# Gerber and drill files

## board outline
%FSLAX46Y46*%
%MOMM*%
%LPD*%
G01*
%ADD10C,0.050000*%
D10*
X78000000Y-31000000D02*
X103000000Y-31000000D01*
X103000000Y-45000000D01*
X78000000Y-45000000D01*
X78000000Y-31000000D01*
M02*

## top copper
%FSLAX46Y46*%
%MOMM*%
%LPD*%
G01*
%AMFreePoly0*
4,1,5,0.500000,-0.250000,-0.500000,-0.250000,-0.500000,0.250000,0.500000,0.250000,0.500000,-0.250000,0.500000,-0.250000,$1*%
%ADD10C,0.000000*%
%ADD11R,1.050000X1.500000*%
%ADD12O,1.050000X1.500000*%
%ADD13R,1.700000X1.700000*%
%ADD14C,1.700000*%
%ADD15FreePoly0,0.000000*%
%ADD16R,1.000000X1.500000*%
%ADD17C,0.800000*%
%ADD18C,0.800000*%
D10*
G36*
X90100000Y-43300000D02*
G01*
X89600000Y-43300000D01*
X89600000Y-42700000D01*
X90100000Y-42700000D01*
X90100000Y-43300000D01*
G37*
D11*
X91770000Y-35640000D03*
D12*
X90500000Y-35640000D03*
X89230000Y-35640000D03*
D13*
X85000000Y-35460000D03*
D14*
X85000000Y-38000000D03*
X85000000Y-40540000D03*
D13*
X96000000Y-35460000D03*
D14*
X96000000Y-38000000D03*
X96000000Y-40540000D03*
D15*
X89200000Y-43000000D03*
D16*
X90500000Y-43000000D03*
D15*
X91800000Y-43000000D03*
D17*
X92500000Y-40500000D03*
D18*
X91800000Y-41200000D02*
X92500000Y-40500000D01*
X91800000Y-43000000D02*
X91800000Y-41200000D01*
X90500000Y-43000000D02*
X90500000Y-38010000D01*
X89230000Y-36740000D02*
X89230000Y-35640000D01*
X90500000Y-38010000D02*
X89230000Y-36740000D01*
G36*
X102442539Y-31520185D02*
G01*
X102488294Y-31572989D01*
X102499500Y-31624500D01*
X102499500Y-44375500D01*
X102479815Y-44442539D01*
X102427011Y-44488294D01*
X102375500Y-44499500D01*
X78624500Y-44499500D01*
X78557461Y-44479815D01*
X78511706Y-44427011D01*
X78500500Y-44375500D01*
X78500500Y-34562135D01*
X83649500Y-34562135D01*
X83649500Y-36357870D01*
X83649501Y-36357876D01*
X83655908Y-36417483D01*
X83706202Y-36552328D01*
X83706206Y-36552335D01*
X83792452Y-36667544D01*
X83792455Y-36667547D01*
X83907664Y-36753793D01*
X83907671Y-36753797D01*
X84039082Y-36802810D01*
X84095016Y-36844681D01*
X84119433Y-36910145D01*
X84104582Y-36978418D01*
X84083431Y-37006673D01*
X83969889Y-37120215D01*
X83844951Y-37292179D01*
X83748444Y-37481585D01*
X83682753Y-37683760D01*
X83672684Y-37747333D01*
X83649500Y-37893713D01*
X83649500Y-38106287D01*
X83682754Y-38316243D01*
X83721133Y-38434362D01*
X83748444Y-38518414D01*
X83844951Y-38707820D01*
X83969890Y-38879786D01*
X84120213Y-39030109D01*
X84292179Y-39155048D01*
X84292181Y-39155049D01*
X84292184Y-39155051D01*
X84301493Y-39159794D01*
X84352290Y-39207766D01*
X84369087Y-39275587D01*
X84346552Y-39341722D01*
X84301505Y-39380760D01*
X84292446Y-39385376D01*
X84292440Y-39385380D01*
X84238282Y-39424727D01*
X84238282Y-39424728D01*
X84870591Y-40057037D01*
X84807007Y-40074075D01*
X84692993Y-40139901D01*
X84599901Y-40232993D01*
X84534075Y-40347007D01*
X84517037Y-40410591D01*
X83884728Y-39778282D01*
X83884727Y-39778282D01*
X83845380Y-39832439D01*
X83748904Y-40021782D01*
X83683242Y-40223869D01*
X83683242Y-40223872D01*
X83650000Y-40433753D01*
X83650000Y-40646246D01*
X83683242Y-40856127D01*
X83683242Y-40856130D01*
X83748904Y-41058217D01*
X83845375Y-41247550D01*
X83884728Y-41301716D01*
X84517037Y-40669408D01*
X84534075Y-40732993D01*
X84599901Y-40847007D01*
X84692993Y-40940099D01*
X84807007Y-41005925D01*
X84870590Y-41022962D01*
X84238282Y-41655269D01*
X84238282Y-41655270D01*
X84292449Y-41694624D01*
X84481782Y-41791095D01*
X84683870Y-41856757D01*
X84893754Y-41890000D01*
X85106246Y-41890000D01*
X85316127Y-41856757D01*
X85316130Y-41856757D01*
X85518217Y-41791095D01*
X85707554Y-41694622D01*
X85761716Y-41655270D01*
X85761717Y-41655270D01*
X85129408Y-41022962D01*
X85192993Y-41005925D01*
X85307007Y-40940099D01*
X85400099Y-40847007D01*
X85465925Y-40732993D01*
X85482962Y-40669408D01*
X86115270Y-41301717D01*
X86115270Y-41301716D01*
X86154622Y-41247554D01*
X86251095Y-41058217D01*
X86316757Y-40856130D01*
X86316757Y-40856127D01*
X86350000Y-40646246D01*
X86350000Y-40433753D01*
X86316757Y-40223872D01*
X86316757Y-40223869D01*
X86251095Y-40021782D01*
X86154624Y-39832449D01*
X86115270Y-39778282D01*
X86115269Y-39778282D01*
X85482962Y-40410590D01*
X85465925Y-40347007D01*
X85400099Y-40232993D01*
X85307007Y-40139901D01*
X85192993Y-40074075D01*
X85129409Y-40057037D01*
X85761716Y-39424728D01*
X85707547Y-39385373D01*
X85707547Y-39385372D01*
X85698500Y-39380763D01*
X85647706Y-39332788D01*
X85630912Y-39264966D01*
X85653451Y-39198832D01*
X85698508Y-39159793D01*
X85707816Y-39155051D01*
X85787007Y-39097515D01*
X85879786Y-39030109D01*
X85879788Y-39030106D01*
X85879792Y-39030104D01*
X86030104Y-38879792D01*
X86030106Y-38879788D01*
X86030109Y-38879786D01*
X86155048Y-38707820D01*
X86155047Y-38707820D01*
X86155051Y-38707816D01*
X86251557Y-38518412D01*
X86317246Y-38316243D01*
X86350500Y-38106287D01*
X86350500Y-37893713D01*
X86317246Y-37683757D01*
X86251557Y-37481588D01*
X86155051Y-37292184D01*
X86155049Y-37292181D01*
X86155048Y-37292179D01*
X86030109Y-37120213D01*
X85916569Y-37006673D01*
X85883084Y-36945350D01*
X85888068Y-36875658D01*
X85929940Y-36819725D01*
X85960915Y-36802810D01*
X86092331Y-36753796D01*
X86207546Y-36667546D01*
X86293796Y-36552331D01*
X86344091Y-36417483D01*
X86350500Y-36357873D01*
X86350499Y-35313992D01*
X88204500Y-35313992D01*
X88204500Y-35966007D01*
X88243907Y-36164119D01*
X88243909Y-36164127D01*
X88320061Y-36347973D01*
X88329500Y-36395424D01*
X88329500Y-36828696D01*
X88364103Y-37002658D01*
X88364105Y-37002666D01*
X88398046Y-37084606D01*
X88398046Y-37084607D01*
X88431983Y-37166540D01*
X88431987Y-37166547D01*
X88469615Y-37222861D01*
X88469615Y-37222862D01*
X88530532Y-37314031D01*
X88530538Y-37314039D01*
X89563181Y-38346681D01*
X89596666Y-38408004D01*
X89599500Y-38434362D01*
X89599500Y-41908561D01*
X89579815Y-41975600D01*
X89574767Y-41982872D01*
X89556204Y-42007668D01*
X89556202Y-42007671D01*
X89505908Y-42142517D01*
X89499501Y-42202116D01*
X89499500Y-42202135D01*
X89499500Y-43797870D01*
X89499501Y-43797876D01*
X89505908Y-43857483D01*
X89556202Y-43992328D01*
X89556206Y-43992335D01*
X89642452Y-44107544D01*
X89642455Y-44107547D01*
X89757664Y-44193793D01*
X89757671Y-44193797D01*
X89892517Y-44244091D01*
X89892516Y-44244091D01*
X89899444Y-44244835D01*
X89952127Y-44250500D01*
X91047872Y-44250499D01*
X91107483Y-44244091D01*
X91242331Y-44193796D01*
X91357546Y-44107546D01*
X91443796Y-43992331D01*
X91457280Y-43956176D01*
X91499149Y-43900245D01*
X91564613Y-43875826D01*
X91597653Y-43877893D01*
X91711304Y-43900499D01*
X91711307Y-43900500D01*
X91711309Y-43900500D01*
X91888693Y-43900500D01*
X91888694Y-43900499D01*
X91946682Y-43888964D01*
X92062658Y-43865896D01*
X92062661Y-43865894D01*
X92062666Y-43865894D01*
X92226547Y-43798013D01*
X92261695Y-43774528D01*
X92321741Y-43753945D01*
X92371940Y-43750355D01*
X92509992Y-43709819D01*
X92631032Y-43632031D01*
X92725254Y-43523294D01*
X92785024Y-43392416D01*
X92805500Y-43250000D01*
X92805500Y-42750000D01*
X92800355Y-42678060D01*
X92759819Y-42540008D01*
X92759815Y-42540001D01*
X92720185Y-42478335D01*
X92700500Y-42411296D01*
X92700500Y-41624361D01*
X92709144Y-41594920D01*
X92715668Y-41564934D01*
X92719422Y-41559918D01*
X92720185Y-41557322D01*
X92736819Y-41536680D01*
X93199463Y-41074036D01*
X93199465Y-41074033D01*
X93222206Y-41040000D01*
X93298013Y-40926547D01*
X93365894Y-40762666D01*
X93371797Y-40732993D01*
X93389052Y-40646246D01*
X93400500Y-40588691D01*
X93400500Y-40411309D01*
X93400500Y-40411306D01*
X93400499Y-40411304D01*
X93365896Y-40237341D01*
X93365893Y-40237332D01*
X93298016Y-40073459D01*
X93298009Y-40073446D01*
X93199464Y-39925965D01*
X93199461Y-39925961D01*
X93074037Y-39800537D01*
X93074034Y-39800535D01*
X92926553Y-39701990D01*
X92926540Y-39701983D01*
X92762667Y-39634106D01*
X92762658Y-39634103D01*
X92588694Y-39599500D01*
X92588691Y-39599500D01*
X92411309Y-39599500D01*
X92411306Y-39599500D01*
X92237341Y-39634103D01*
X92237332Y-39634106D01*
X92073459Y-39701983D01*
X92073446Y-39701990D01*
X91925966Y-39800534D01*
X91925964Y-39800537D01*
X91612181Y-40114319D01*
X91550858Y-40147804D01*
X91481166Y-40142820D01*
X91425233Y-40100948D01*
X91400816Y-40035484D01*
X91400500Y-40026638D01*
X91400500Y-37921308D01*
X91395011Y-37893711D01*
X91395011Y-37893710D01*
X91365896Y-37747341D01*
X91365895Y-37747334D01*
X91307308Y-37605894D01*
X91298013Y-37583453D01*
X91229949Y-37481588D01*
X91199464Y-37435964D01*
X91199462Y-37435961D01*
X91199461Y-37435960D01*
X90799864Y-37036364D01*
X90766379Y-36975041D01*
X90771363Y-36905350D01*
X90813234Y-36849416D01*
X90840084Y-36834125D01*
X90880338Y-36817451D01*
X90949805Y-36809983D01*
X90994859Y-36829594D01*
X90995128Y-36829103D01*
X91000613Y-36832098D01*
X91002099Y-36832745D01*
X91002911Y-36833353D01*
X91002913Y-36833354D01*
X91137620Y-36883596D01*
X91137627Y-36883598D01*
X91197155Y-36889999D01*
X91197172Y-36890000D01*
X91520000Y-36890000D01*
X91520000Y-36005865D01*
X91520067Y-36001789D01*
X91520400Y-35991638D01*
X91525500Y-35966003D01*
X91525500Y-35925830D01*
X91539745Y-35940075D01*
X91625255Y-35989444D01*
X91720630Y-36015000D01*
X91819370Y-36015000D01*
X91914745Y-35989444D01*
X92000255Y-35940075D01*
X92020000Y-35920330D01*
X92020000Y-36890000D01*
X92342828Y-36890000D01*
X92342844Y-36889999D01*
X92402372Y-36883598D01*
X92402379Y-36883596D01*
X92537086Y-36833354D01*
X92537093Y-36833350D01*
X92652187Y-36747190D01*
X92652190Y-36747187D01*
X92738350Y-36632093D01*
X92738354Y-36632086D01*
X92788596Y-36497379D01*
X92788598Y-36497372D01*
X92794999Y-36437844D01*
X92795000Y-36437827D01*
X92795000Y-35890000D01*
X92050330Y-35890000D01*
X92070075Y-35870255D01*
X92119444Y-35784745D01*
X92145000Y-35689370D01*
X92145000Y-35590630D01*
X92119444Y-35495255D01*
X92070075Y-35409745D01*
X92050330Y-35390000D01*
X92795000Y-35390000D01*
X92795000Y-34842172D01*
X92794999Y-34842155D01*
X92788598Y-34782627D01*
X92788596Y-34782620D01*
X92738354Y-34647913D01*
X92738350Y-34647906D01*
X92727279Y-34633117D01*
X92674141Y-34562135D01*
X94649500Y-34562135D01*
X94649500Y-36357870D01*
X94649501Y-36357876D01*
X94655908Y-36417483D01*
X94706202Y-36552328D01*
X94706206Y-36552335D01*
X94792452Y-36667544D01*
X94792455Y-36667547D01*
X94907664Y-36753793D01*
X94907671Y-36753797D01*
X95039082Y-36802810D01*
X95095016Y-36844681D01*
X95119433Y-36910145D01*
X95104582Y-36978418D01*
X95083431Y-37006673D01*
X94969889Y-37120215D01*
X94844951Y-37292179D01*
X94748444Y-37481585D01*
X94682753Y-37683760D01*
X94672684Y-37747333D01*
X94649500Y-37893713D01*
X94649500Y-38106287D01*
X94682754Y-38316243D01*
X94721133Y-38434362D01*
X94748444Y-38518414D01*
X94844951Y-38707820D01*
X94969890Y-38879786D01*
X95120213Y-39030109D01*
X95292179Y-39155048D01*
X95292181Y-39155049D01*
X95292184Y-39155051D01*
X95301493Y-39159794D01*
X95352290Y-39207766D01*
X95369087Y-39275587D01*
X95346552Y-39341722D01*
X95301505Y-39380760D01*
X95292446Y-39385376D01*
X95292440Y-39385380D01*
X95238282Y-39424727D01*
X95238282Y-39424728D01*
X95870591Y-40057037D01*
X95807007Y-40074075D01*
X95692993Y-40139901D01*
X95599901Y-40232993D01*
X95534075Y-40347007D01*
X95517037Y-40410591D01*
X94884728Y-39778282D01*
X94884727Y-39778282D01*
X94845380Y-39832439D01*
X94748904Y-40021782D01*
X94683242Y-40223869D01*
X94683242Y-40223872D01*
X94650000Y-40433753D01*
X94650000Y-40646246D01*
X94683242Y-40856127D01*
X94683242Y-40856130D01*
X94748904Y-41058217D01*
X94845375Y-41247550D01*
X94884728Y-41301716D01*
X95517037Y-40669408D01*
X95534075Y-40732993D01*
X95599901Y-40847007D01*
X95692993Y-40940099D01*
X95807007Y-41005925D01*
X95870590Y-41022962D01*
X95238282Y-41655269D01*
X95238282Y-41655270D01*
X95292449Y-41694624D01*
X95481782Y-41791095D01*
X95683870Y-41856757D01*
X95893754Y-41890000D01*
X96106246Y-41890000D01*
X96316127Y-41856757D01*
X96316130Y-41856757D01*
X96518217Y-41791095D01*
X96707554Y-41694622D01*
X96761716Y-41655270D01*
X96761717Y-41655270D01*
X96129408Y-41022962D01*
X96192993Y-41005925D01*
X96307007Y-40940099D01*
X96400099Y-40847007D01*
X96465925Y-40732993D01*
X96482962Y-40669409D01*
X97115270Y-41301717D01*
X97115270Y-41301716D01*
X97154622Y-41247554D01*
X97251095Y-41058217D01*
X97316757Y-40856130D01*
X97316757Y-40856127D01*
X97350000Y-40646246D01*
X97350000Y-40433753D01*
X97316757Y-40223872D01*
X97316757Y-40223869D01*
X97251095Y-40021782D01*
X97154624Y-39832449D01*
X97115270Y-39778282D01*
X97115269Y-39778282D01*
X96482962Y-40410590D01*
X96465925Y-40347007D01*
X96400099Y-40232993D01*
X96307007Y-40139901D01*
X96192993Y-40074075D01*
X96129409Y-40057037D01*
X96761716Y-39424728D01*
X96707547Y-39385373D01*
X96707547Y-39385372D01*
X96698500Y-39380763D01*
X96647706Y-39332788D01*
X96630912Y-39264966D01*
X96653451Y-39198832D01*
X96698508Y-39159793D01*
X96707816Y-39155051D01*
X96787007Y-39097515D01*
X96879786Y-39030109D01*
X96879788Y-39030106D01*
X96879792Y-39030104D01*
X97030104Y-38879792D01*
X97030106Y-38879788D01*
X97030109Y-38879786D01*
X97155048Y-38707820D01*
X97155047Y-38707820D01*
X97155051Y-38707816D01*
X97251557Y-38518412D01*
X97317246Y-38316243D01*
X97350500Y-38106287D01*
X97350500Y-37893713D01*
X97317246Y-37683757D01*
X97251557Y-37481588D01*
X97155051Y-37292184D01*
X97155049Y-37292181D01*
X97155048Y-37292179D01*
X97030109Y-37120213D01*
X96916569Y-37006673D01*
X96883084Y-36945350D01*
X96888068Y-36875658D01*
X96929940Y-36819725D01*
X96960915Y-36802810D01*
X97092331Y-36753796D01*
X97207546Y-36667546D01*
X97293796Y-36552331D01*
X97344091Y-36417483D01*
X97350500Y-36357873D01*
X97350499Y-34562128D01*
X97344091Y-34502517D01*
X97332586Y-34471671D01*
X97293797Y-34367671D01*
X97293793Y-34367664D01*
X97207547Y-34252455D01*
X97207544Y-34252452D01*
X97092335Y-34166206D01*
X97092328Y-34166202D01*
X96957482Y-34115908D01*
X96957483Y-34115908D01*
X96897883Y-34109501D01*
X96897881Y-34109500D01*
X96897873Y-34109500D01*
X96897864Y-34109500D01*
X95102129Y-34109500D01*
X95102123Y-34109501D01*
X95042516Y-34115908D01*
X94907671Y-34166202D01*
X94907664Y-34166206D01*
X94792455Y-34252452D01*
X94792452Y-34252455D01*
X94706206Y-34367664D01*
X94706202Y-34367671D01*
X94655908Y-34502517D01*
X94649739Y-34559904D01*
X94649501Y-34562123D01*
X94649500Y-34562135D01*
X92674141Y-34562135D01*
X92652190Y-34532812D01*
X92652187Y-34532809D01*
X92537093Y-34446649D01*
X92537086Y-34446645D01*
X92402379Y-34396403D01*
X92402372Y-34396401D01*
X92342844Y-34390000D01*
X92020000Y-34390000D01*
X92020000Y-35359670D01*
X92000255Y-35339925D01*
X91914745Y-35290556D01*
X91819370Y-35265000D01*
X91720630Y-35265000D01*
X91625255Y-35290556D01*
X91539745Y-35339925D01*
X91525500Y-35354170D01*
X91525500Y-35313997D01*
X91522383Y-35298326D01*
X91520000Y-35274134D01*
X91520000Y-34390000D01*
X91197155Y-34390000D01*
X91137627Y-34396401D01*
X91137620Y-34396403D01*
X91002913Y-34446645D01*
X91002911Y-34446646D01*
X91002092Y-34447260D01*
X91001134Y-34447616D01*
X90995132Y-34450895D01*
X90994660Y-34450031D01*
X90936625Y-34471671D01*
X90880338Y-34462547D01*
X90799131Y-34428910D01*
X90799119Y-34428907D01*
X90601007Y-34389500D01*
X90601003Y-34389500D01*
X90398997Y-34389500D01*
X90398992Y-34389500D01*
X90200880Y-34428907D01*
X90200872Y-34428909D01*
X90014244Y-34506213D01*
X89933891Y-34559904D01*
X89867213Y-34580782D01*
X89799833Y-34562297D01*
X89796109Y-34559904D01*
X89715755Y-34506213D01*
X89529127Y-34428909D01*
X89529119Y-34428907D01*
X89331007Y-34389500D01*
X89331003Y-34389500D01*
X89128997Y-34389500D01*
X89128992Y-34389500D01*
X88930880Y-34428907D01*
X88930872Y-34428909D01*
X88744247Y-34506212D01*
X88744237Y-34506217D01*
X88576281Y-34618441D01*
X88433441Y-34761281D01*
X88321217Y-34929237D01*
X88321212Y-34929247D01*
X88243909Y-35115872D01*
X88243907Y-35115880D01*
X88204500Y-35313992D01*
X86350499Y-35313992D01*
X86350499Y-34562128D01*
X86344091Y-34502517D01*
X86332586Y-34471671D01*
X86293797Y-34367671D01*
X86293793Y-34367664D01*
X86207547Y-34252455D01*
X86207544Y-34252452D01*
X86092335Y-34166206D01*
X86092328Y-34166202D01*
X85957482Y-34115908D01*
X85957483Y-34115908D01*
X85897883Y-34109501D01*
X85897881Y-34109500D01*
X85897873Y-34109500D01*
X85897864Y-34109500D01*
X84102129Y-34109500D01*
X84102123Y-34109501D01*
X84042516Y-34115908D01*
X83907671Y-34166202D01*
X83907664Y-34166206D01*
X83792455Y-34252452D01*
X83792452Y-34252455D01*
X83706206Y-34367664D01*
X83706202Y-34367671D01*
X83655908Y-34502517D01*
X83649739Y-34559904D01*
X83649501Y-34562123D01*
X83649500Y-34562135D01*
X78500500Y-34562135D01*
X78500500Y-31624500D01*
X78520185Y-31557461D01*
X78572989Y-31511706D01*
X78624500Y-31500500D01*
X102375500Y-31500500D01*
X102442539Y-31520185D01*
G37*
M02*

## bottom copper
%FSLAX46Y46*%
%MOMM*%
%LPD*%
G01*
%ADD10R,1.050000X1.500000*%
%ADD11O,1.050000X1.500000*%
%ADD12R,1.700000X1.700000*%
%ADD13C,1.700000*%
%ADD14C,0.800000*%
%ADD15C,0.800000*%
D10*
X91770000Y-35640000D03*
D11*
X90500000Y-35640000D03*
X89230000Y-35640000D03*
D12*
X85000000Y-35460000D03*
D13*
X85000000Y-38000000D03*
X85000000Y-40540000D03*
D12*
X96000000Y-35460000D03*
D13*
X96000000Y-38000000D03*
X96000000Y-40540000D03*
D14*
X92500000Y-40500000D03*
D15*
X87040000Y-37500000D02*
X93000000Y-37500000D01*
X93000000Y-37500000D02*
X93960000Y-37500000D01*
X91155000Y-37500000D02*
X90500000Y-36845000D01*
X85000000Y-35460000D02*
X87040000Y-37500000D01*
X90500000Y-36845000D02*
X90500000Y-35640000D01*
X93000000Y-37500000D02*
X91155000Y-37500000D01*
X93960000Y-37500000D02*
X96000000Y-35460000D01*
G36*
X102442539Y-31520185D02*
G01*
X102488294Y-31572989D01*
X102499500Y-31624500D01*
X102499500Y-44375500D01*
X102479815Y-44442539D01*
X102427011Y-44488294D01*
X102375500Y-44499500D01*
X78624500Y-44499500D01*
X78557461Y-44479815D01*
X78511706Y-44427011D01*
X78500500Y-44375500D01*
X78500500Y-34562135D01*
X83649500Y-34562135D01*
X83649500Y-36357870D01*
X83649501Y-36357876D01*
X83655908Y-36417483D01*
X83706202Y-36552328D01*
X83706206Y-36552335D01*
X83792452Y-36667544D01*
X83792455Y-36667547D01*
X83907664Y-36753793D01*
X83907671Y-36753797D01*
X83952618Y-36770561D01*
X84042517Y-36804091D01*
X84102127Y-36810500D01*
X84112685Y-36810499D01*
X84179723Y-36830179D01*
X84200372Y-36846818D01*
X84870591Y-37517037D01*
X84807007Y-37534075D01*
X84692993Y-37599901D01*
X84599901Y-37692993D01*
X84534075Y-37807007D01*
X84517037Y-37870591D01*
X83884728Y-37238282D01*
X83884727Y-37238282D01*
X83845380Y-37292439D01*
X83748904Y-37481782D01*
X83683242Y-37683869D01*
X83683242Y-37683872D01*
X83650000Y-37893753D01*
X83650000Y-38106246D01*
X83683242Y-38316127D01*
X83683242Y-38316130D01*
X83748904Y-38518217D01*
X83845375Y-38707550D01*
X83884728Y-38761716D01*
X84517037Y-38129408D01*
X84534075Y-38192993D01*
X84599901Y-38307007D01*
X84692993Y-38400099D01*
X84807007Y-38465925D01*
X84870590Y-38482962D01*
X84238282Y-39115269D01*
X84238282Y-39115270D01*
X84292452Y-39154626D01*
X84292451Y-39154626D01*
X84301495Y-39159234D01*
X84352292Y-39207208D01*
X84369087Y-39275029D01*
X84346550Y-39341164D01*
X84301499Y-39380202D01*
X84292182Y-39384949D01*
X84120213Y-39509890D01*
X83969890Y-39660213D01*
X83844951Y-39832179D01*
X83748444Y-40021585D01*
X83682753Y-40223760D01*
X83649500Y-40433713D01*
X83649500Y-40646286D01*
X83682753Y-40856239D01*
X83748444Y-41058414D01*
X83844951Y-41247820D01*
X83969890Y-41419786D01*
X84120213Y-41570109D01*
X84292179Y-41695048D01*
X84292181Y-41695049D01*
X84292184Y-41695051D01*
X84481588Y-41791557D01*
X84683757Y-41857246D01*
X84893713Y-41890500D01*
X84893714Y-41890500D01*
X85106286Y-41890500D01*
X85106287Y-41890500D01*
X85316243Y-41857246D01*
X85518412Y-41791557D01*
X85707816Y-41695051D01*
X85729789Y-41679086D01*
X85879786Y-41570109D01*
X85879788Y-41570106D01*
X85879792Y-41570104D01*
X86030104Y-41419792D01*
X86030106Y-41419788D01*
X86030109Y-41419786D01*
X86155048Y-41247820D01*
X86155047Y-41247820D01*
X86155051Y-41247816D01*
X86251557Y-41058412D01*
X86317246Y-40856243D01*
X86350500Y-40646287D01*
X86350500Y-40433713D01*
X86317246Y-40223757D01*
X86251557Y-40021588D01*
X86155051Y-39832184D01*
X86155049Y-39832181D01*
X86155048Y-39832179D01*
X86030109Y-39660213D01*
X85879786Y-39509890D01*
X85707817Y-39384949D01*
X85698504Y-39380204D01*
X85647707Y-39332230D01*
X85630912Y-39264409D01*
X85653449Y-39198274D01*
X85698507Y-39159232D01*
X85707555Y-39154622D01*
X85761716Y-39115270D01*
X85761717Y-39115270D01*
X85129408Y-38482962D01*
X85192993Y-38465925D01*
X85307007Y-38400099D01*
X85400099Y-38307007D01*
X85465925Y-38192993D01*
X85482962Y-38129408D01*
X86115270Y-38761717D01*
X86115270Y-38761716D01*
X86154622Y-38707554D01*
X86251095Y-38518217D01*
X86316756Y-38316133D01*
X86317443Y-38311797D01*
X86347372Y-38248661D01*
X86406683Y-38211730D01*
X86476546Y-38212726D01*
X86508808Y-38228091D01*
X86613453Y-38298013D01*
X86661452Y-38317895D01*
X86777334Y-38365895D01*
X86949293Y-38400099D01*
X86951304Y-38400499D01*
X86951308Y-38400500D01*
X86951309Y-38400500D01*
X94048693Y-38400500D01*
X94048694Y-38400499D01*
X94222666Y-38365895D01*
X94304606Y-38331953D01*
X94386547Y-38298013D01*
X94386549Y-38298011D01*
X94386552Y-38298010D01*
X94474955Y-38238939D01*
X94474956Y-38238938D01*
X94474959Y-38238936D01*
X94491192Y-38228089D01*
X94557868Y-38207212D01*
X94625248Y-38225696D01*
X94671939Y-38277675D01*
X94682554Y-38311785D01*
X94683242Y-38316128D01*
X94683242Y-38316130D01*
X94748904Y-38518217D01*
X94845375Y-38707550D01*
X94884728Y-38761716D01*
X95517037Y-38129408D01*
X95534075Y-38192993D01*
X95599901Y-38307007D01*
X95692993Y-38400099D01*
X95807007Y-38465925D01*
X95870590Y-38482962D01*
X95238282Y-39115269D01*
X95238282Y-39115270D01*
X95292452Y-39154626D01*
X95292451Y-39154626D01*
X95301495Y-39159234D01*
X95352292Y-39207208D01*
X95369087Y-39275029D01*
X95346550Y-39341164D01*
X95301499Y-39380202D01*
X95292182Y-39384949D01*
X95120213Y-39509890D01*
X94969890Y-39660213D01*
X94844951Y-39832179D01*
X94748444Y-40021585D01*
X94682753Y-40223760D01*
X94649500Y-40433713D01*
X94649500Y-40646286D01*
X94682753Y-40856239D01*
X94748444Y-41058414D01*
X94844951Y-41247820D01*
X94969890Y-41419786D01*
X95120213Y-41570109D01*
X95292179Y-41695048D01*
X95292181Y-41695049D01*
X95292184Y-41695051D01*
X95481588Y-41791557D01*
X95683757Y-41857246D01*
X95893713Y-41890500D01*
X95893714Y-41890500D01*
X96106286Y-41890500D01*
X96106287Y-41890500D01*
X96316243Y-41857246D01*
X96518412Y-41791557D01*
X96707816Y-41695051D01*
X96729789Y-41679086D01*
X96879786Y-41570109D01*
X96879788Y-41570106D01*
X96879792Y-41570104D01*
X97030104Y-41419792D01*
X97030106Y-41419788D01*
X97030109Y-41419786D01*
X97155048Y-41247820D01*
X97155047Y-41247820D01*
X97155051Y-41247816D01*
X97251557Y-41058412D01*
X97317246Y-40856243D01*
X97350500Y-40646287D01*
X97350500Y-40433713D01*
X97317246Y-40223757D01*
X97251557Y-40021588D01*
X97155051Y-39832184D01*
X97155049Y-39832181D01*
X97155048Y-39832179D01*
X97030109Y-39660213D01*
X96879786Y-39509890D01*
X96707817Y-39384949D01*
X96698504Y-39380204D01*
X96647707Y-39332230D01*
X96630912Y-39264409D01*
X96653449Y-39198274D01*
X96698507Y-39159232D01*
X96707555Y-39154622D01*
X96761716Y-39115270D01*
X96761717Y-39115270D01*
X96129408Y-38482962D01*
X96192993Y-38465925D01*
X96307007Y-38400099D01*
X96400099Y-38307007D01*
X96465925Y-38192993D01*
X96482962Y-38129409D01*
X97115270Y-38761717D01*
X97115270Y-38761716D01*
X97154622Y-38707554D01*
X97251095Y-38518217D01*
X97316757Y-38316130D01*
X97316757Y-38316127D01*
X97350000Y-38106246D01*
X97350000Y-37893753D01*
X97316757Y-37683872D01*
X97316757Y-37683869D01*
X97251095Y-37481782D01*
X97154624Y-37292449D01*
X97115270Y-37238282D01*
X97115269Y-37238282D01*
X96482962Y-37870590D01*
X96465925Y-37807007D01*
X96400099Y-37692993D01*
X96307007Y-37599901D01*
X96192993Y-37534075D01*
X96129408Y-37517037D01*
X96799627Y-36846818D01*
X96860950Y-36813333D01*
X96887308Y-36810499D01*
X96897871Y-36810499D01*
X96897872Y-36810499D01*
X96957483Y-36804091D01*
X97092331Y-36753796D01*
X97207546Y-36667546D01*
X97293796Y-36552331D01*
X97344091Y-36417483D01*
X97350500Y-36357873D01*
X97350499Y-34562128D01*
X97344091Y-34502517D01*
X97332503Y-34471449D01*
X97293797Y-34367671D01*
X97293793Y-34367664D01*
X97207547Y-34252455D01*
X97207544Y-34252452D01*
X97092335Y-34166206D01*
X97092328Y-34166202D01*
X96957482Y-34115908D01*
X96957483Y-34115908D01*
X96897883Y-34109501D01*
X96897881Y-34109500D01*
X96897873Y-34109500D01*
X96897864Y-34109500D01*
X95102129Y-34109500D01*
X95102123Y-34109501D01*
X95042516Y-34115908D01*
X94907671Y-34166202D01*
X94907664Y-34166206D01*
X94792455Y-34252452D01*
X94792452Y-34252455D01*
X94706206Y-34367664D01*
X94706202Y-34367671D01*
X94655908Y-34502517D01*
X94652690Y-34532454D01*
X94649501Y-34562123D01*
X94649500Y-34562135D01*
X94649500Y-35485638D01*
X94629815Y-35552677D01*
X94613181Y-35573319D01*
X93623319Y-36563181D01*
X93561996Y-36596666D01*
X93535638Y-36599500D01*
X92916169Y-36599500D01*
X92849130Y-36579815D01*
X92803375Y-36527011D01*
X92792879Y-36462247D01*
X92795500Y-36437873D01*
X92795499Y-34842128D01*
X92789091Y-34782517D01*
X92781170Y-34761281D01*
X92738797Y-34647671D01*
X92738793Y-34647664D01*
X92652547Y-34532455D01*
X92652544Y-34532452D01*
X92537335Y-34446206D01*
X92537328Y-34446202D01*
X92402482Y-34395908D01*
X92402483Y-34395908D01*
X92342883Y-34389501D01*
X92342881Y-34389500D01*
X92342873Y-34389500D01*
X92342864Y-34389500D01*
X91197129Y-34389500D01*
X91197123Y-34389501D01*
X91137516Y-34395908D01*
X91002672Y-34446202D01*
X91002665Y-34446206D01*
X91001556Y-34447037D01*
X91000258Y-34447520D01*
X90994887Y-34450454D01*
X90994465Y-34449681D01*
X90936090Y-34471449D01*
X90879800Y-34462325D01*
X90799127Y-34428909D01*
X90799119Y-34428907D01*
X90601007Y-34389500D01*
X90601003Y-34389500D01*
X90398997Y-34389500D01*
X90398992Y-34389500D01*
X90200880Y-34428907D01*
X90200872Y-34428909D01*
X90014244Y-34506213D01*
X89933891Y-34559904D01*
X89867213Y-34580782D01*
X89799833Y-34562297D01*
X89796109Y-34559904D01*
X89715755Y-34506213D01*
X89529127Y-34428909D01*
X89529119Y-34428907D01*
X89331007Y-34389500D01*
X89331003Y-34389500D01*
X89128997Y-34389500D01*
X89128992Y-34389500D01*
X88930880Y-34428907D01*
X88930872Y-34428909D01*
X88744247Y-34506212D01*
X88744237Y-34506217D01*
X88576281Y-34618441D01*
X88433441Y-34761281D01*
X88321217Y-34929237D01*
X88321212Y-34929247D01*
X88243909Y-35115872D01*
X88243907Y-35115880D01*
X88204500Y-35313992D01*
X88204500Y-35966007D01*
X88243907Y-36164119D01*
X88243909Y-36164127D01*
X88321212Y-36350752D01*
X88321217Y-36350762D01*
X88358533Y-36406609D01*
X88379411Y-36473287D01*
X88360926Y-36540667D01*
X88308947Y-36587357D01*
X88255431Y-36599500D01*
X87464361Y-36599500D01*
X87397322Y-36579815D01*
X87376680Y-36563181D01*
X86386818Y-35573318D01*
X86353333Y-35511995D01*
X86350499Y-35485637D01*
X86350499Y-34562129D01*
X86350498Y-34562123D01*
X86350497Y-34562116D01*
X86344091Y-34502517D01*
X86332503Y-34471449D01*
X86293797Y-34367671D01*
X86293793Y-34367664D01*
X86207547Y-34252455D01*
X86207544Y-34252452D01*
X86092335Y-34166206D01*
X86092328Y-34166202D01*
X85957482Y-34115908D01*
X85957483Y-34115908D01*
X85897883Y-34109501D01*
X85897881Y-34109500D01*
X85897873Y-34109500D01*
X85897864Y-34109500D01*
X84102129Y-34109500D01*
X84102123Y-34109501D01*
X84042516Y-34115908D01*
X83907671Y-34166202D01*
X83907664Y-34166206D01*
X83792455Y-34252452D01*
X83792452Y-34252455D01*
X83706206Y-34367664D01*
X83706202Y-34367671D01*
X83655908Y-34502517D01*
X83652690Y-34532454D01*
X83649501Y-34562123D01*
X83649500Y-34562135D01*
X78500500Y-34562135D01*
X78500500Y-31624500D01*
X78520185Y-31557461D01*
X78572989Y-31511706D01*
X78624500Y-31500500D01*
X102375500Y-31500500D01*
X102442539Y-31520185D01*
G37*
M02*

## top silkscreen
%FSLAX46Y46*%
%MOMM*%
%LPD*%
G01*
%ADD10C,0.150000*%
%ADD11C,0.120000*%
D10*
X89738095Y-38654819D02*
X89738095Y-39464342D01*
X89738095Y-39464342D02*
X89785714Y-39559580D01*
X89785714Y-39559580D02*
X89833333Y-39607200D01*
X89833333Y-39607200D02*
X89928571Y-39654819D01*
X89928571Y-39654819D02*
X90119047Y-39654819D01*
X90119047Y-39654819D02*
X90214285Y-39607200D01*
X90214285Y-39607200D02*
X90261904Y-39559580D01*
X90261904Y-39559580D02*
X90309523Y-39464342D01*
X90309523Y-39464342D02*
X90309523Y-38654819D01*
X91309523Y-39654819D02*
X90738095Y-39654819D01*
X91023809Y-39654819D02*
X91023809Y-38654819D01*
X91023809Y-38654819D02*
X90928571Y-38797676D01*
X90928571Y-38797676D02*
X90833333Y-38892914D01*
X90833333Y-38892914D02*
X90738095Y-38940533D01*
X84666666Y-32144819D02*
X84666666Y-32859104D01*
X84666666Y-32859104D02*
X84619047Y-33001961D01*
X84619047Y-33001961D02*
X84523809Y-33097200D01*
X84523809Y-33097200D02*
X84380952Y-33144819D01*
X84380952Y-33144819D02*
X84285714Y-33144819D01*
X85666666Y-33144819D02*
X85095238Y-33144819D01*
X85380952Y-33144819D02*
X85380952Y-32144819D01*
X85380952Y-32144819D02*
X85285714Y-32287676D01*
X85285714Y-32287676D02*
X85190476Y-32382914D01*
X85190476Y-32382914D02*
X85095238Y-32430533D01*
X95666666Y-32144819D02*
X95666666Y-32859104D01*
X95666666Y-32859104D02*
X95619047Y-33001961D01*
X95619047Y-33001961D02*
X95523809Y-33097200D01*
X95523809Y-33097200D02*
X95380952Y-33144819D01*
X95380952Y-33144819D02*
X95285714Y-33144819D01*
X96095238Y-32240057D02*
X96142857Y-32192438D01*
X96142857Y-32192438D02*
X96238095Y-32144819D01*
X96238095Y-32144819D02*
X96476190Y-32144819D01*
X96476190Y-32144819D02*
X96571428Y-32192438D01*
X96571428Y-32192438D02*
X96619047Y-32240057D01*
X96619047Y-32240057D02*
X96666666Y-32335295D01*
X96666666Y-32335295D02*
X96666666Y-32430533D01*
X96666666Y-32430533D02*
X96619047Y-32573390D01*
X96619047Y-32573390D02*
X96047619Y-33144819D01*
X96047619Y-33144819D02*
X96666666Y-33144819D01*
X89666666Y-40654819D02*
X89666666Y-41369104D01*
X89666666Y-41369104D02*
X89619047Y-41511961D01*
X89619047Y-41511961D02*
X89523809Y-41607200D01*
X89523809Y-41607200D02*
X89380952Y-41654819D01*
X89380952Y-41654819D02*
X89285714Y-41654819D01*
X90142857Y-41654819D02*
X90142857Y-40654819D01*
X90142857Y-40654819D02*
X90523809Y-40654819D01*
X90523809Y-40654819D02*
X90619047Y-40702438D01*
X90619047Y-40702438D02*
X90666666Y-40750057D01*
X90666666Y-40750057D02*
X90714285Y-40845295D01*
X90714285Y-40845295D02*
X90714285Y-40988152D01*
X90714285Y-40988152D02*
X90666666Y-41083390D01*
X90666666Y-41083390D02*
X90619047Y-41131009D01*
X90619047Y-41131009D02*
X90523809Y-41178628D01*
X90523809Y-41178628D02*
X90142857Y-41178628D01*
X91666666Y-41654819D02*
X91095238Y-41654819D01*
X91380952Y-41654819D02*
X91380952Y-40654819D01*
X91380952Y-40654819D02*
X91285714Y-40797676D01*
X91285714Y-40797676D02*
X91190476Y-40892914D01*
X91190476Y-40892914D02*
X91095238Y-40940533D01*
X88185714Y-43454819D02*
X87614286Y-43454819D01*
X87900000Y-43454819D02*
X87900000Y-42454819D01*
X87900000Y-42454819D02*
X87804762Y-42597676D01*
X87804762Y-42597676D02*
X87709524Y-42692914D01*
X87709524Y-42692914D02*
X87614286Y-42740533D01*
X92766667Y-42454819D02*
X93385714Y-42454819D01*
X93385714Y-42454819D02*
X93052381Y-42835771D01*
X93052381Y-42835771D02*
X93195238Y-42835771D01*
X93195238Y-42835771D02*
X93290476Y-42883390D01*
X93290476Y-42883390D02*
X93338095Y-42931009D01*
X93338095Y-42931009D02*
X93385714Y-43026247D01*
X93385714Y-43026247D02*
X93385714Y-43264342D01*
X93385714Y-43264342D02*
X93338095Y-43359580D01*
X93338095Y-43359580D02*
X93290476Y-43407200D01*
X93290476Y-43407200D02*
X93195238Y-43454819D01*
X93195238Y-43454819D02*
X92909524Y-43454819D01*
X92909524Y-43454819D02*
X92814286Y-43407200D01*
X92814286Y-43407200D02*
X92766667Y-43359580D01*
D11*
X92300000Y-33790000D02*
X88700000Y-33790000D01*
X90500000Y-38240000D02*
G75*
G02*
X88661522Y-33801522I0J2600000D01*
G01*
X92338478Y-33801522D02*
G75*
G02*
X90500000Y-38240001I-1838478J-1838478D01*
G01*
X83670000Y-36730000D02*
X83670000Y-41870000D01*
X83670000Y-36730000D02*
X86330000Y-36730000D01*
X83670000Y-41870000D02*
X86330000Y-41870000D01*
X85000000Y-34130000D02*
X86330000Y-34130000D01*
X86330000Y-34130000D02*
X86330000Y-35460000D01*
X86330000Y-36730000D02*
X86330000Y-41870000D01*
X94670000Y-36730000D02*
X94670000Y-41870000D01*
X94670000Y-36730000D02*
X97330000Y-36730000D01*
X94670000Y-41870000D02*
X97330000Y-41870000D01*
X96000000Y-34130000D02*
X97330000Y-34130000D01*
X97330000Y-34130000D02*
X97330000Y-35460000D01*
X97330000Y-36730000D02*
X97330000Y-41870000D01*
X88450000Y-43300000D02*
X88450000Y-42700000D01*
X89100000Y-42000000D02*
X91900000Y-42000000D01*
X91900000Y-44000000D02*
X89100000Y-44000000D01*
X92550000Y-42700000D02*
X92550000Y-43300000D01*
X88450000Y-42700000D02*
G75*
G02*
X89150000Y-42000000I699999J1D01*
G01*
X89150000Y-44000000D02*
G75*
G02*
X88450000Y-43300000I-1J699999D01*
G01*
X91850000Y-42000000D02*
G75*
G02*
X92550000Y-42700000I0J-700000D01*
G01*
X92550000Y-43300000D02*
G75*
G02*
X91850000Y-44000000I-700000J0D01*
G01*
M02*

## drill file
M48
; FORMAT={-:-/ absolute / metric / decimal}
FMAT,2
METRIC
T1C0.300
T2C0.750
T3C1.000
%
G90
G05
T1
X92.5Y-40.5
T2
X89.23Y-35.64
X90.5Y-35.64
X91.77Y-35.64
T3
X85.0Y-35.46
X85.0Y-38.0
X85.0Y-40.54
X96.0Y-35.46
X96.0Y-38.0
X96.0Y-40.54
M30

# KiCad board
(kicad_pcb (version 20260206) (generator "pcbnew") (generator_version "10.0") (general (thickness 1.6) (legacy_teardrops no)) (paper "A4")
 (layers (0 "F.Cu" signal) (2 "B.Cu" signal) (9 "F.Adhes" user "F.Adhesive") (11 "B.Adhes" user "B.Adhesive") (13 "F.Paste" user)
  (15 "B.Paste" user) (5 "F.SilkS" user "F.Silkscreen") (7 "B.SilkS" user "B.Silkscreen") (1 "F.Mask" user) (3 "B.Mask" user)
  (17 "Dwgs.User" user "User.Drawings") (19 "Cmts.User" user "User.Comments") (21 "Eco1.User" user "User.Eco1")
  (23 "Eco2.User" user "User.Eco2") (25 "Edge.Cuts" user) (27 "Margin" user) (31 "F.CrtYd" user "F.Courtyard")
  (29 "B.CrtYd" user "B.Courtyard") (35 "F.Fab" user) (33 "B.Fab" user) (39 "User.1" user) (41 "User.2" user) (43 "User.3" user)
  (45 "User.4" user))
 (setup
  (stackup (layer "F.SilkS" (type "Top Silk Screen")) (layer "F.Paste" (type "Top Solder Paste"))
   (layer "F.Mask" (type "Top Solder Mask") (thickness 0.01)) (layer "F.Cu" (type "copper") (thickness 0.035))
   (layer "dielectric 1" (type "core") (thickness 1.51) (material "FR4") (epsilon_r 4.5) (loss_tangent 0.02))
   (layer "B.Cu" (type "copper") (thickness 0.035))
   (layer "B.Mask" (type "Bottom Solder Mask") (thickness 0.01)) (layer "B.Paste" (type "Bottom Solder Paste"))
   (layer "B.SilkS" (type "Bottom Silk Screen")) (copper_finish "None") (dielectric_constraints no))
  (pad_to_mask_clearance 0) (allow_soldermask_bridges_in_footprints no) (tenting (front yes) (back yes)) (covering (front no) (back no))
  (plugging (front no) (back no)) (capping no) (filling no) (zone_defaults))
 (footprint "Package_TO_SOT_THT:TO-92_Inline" (layer "F.Cu") (at 91.77 35.64 180)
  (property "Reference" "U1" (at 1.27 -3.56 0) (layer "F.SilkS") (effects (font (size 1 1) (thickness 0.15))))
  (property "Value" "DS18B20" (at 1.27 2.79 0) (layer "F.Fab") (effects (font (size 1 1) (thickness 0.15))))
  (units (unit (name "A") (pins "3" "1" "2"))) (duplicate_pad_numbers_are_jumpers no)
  (fp_line (start -0.53 1.85) (end 3.07 1.85) (stroke (width 0.12) (type solid)) (layer "F.SilkS"))
  (fp_arc (start 1.27 -2.6) (mid 3.672087 -0.994977) (end 3.108478 1.838478) (stroke (width 0.12) (type solid)) (layer "F.SilkS"))
  (fp_arc (start -0.568478 1.838478) (mid -1.132087 -0.994977) (end 1.27 -2.6) (stroke (width 0.12) (type solid)) (layer "F.SilkS"))
  (pad "1" thru_hole rect (at 0 0 180) (size 1.05 1.5) (drill 0.75) (layers "*.Cu" "*.Mask") (remove_unused_layers no) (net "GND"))
  (pad "2" thru_hole oval (at 1.27 0 180) (size 1.05 1.5) (drill 0.75) (layers "*.Cu" "*.Mask") (remove_unused_layers no) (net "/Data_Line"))
  (pad "3" thru_hole oval (at 2.54 0 180) (size 1.05 1.5) (drill 0.75) (layers "*.Cu" "*.Mask") (remove_unused_layers no)
   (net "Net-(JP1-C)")))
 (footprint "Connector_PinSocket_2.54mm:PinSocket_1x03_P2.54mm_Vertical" (layer "F.Cu") (at 85 35.46)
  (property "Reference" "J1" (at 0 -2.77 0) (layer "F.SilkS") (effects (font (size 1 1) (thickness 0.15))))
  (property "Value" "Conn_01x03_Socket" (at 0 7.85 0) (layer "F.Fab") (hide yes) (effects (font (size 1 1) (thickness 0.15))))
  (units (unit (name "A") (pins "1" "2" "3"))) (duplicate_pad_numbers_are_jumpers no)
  (fp_line (start -1.33 1.27) (end -1.33 6.41) (stroke (width 0.12) (type solid)) (layer "F.SilkS"))
  (fp_line (start -1.33 1.27) (end 1.33 1.27) (stroke (width 0.12) (type solid)) (layer "F.SilkS"))
  (fp_line (start -1.33 6.41) (end 1.33 6.41) (stroke (width 0.12) (type solid)) (layer "F.SilkS"))
  (fp_line (start 0 -1.33) (end 1.33 -1.33) (stroke (width 0.12) (type solid)) (layer "F.SilkS"))
  (fp_line (start 1.33 -1.33) (end 1.33 0) (stroke (width 0.12) (type solid)) (layer "F.SilkS"))
  (fp_line (start 1.33 1.27) (end 1.33 6.41) (stroke (width 0.12) (type solid)) (layer "F.SilkS"))
  (pad "1" thru_hole rect (at 0 0) (size 1.7 1.7) (drill 1) (layers "*.Cu" "*.Mask") (remove_unused_layers no) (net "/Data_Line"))
  (pad "2" thru_hole circle (at 0 2.54) (size 1.7 1.7) (drill 1) (layers "*.Cu" "*.Mask") (remove_unused_layers no) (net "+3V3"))
  (pad "3" thru_hole circle (at 0 5.08) (size 1.7 1.7) (drill 1) (layers "*.Cu" "*.Mask") (remove_unused_layers no) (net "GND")))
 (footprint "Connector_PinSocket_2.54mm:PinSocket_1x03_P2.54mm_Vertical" (layer "F.Cu") (at 96 35.46)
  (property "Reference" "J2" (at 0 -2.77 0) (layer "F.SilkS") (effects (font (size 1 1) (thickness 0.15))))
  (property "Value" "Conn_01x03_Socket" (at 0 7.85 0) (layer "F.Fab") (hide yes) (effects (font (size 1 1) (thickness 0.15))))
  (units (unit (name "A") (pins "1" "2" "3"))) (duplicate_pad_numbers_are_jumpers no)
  (fp_line (start -1.33 1.27) (end -1.33 6.41) (stroke (width 0.12) (type solid)) (layer "F.SilkS"))
  (fp_line (start -1.33 1.27) (end 1.33 1.27) (stroke (width 0.12) (type solid)) (layer "F.SilkS"))
  (fp_line (start -1.33 6.41) (end 1.33 6.41) (stroke (width 0.12) (type solid)) (layer "F.SilkS"))
  (fp_line (start 0 -1.33) (end 1.33 -1.33) (stroke (width 0.12) (type solid)) (layer "F.SilkS"))
  (fp_line (start 1.33 -1.33) (end 1.33 0) (stroke (width 0.12) (type solid)) (layer "F.SilkS"))
  (fp_line (start 1.33 1.27) (end 1.33 6.41) (stroke (width 0.12) (type solid)) (layer "F.SilkS"))
  (pad "1" thru_hole rect (at 0 0) (size 1.7 1.7) (drill 1) (layers "*.Cu" "*.Mask") (remove_unused_layers no) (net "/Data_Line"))
  (pad "2" thru_hole circle (at 0 2.54) (size 1.7 1.7) (drill 1) (layers "*.Cu" "*.Mask") (remove_unused_layers no) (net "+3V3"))
  (pad "3" thru_hole circle (at 0 5.08) (size 1.7 1.7) (drill 1) (layers "*.Cu" "*.Mask") (remove_unused_layers no) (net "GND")))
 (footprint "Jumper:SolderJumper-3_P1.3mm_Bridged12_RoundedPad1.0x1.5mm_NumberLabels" (layer "F.Cu") (at 90.5 43)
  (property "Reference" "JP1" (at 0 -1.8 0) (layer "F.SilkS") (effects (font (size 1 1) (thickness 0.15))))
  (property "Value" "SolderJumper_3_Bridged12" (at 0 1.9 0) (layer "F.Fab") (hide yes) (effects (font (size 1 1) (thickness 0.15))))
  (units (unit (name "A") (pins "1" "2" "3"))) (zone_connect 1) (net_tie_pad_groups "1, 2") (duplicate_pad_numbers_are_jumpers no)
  (fp_poly (pts (xy -0.9 -0.3) (xy -0.4 -0.3) (xy -0.4 0.3) (xy -0.9 0.3)) (stroke (width 0) (type solid)) (fill yes) (layer "F.Cu"))
  (fp_line (start -2.05 0.3) (end -2.05 -0.3) (stroke (width 0.12) (type solid)) (layer "F.SilkS"))
  (fp_line (start -1.4 -1) (end 1.4 -1) (stroke (width 0.12) (type solid)) (layer "F.SilkS"))
  (fp_line (start 1.4 1) (end -1.4 1) (stroke (width 0.12) (type solid)) (layer "F.SilkS"))
  (fp_line (start 2.05 -0.3) (end 2.05 0.3) (stroke (width 0.12) (type solid)) (layer "F.SilkS"))
  (fp_arc (start -2.05 -0.3) (mid -1.844975 -0.794975) (end -1.35 -1) (stroke (width 0.12) (type solid)) (layer "F.SilkS"))
  (fp_arc (start -1.35 1) (mid -1.844975 0.794975) (end -2.05 0.3) (stroke (width 0.12) (type solid)) (layer "F.SilkS"))
  (fp_arc (start 1.35 -1) (mid 1.844975 -0.794975) (end 2.05 -0.3) (stroke (width 0.12) (type solid)) (layer "F.SilkS"))
  (fp_arc (start 2.05 0.3) (mid 1.844975 0.794975) (end 1.35 1) (stroke (width 0.12) (type solid)) (layer "F.SilkS"))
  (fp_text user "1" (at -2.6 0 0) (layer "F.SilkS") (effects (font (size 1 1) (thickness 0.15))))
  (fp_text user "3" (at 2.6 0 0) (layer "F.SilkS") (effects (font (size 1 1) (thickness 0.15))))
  (pad "1" smd custom (at -1.3 0) (size 1 0.5) (layers "F.Cu" "F.Mask") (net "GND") (zone_connect 2) (thermal_bridge_angle 45)
   (options (clearance outline) (anchor rect)) (primitives))
  (pad "2" smd rect (at 0 0) (size 1 1.5) (layers "F.Cu" "F.Mask") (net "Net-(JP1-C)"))
  (pad "3" smd custom (at 1.3 0) (size 1 0.5) (layers "F.Cu" "F.Mask") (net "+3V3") (zone_connect 2) (thermal_bridge_angle 45)
   (options (clearance outline) (anchor rect)) (primitives)))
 (gr_rect (start 78 31) (end 103 45) (stroke (width 0.05) (type default)) (fill no) (layer "Edge.Cuts"))
 (segment (start 87.04 37.5) (end 93 37.5) (width 0.8) (layer "B.Cu") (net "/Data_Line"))
 (segment (start 93 37.5) (end 93.96 37.5) (width 0.8) (layer "B.Cu") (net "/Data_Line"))
 (segment (start 91.155 37.5) (end 90.5 36.845) (width 0.8) (layer "B.Cu") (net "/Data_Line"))
 (segment (start 85 35.46) (end 87.04 37.5) (width 0.8) (layer "B.Cu") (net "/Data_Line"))
 (segment (start 90.5 36.845) (end 90.5 35.64) (width 0.8) (layer "B.Cu") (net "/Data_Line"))
 (segment (start 93 37.5) (end 91.155 37.5) (width 0.8) (layer "B.Cu") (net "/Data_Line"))
 (segment (start 93.96 37.5) (end 96 35.46) (width 0.8) (layer "B.Cu") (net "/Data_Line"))
 (segment (start 91.8 41.2) (end 92.5 40.5) (width 0.8) (layer "F.Cu") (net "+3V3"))
 (segment (start 91.8 43) (end 91.8 41.2) (width 0.8) (layer "F.Cu") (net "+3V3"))
 (via (at 92.5 40.5) (size 0.8) (drill 0.3) (layers "F.Cu" "B.Cu") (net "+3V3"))
 (segment (start 90.5 43) (end 90.5 38.01) (width 0.8) (layer "F.Cu") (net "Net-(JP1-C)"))
 (segment (start 89.23 36.74) (end 89.23 35.64) (width 0.8) (layer "F.Cu") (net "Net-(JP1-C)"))
 (segment (start 90.5 38.01) (end 89.23 36.74) (width 0.8) (layer "F.Cu") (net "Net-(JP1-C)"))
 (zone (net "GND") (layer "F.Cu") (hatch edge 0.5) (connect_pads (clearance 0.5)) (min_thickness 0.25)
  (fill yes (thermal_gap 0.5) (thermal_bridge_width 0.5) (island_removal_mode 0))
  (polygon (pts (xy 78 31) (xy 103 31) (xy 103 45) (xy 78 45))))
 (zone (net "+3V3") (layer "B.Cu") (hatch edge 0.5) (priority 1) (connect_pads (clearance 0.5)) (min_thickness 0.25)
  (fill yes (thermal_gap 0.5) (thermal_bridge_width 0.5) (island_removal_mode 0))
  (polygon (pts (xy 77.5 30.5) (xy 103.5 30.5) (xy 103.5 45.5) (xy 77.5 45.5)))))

